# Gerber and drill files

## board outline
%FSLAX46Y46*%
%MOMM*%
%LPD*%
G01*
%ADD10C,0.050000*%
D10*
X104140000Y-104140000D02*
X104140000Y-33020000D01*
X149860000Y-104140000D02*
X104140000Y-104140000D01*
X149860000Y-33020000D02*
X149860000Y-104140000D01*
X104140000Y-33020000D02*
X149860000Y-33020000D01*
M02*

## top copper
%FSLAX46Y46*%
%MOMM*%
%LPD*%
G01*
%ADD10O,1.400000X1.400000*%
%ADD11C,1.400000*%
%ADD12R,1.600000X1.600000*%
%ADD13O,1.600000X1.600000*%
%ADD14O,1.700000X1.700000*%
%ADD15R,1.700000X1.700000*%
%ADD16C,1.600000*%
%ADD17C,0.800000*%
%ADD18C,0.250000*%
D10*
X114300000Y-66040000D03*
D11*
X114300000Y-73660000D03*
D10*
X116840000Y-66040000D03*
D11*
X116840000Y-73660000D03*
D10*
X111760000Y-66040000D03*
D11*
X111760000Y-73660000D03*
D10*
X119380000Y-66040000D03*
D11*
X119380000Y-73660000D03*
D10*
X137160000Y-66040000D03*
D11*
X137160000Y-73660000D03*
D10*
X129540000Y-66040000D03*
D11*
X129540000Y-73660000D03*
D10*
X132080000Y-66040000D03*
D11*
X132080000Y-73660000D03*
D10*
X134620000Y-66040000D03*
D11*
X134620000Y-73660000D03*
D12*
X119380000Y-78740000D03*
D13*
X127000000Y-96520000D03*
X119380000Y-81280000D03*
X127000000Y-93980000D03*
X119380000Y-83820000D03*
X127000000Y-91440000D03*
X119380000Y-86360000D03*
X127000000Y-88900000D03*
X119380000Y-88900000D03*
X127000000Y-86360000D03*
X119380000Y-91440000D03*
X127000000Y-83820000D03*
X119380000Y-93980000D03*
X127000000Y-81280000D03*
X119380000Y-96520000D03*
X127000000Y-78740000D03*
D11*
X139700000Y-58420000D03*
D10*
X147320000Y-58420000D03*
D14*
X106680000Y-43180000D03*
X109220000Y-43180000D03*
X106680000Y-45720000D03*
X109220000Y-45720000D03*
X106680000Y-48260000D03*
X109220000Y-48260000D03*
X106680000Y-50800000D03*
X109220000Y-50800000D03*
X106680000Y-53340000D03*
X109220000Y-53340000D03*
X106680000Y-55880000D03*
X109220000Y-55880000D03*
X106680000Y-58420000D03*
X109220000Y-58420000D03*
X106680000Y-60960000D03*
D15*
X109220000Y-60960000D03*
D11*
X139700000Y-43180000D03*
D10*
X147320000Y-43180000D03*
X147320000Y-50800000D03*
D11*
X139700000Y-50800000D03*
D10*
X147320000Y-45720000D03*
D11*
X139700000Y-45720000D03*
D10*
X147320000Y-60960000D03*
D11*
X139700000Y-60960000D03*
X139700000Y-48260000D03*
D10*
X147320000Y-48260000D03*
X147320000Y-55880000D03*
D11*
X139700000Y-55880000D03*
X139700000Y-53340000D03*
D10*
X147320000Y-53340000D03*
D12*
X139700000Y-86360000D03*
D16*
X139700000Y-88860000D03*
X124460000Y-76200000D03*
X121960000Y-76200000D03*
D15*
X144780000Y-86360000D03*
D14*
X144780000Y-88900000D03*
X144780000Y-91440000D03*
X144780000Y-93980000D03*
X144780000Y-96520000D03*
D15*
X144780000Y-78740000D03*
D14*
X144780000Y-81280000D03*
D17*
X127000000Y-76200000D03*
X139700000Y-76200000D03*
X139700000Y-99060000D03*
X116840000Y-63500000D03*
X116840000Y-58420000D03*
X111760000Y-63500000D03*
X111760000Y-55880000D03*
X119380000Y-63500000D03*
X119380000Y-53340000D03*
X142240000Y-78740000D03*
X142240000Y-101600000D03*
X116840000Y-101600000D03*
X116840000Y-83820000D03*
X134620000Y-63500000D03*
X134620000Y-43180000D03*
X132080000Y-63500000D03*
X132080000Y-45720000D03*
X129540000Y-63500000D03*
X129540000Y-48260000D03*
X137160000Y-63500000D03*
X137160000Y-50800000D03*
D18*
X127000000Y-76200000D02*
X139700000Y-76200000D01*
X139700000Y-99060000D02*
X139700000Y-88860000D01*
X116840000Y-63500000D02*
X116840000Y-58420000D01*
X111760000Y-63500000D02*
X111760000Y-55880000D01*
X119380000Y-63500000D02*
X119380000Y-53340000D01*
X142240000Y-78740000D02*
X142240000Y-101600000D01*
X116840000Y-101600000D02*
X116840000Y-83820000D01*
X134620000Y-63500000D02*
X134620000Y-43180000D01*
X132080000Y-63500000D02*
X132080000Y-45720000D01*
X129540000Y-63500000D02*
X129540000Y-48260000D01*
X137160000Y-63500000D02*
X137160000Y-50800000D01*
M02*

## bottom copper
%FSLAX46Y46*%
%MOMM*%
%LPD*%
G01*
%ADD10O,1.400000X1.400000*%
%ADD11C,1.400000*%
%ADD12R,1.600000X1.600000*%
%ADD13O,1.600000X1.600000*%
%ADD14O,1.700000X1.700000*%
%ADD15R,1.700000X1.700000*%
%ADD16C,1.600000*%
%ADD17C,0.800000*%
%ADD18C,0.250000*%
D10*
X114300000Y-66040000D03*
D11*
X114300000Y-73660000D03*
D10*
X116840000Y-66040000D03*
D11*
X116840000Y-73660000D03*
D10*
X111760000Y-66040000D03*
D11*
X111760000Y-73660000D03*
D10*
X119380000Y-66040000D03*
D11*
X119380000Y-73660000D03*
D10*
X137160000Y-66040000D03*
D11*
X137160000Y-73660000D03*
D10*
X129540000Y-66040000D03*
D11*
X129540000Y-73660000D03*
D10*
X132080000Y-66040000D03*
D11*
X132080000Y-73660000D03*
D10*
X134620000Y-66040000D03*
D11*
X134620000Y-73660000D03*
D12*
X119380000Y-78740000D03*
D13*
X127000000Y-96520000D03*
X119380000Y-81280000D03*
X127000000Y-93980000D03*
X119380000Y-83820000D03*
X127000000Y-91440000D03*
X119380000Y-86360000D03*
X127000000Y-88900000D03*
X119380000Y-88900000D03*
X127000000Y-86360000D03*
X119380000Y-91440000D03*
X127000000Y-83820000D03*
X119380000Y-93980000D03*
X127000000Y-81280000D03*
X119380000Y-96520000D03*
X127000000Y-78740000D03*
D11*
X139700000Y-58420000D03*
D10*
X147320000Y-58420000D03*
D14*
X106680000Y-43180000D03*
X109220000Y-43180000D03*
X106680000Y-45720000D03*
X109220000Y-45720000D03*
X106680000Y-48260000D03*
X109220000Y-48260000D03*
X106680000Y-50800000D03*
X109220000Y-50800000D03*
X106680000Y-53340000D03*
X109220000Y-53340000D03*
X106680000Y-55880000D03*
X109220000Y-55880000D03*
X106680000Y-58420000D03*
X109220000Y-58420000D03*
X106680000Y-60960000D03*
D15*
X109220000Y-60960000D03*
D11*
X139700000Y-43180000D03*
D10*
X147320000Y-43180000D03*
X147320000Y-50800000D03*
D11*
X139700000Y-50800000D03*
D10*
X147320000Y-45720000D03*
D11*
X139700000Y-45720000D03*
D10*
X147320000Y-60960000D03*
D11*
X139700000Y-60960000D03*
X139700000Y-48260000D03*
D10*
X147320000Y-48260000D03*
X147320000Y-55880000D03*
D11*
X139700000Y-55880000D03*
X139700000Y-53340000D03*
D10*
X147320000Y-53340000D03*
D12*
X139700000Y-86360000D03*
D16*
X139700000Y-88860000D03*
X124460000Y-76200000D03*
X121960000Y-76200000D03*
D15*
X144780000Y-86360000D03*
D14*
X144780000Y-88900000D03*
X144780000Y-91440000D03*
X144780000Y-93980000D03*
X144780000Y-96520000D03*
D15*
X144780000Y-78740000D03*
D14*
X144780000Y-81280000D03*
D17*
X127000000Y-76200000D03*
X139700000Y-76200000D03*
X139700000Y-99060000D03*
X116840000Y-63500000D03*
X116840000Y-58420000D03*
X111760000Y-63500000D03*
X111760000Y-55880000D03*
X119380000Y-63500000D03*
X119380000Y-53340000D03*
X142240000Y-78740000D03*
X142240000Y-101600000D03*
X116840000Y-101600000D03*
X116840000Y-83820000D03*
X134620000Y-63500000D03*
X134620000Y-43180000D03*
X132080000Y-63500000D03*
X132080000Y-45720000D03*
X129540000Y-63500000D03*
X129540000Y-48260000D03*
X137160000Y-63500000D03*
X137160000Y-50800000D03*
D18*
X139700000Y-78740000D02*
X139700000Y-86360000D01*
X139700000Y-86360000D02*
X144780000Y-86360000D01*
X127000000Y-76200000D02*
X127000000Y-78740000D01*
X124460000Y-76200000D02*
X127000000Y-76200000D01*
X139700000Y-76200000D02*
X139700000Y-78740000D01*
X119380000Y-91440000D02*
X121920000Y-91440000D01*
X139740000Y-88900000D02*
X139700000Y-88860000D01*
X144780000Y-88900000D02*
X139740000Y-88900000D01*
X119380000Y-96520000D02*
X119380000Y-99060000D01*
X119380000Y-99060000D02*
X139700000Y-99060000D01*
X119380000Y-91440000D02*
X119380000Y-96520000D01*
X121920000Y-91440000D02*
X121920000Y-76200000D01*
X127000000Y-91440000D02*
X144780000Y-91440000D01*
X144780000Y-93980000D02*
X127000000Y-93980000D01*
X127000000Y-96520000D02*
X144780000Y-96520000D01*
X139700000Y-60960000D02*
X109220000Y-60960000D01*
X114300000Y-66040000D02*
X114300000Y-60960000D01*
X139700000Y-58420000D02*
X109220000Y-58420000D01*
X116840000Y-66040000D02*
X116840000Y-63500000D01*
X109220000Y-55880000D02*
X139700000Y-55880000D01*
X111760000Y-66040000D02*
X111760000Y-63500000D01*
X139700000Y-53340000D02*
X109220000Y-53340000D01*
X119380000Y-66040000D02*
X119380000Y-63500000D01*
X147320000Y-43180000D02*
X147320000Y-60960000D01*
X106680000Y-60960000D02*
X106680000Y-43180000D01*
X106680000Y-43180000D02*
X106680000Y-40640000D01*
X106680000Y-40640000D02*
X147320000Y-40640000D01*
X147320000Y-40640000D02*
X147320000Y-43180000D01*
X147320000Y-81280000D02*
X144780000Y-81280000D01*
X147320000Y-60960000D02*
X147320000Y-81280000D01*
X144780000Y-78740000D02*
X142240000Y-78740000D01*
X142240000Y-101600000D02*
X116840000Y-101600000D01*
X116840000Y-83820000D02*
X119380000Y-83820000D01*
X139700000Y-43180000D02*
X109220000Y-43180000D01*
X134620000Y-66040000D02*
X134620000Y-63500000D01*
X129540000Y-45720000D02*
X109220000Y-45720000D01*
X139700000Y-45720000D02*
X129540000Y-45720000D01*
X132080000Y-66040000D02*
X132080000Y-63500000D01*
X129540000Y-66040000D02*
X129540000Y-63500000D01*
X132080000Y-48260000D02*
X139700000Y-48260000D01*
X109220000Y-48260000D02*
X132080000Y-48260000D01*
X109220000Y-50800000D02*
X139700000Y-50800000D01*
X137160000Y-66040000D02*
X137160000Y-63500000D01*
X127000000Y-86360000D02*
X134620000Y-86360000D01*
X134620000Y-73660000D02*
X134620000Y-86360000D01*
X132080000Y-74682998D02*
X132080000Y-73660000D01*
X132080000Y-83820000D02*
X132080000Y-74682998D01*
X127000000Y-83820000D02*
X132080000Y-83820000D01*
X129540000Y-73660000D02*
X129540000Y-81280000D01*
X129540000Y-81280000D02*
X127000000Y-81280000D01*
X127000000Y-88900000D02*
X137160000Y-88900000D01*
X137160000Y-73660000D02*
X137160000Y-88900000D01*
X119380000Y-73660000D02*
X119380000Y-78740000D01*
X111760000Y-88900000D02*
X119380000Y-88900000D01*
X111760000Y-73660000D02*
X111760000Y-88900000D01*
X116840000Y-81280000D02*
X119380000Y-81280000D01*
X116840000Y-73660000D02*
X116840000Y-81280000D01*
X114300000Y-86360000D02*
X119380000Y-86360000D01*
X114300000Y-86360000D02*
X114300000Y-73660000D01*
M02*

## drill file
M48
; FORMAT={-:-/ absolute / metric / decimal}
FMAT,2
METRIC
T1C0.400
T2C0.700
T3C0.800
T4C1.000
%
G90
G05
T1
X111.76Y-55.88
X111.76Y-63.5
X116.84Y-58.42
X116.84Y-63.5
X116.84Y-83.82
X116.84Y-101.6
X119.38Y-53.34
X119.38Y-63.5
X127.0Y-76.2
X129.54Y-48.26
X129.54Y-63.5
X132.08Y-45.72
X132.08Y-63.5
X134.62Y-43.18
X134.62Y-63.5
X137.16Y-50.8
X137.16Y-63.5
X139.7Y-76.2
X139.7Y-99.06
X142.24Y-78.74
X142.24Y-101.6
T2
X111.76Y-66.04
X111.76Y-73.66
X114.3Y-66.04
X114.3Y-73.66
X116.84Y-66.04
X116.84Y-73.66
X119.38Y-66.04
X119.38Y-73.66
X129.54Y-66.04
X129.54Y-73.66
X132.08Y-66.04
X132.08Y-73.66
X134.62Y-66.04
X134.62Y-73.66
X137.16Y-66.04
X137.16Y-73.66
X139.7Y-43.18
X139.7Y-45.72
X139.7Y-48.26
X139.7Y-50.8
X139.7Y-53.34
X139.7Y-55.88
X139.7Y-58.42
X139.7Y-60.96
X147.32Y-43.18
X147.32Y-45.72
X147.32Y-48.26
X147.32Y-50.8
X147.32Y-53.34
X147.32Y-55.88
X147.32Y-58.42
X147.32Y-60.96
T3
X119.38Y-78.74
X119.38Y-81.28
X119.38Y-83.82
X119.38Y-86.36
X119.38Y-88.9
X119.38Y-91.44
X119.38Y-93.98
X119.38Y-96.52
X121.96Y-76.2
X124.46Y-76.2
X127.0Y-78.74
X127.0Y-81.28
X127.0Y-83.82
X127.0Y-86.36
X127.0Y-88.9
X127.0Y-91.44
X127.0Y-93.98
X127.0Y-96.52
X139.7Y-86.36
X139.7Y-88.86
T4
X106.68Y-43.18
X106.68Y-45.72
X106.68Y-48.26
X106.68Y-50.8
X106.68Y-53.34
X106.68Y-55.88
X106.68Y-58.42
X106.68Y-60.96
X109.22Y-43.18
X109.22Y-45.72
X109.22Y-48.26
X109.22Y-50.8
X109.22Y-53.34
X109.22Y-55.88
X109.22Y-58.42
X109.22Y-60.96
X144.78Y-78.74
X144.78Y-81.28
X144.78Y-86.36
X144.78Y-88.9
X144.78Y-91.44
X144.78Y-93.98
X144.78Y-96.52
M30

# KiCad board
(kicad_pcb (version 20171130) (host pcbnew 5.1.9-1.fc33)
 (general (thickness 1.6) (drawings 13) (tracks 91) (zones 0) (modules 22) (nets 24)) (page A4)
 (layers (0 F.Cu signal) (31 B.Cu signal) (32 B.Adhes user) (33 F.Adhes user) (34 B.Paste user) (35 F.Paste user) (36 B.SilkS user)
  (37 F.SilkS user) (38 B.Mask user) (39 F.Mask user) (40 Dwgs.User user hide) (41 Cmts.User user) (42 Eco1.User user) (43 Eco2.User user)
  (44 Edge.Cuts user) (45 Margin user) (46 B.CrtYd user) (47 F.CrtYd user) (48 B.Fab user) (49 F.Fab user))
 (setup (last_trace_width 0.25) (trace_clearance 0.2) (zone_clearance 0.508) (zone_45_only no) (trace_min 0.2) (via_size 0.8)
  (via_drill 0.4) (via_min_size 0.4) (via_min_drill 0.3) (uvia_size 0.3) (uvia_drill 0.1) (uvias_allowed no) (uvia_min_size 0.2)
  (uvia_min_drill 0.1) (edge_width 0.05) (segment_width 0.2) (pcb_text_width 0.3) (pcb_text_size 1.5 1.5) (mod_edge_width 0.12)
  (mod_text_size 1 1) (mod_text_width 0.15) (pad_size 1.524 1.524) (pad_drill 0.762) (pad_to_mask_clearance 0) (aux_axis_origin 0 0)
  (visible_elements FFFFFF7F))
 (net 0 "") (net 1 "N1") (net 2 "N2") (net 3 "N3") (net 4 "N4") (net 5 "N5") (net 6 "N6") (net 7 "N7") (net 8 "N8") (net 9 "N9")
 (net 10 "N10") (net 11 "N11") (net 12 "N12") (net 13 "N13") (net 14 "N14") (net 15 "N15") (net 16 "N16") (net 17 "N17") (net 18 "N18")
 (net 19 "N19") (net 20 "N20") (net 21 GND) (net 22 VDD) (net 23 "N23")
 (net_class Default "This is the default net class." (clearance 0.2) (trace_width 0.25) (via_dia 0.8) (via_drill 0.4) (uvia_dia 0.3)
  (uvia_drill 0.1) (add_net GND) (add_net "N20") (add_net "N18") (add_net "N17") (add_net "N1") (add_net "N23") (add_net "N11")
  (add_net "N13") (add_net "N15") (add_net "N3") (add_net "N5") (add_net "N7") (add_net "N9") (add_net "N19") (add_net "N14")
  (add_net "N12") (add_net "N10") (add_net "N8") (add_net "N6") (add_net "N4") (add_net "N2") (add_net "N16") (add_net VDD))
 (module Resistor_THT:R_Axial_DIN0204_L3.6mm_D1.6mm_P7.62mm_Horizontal (layer F.Cu) (at 114.3 73.66 90)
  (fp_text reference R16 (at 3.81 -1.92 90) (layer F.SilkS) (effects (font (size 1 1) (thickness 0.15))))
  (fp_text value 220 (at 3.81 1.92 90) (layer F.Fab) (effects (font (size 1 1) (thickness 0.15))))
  (pad 2 thru_hole oval (at 7.62 0 90) (size 1.4 1.4) (drill 0.7) (layers *.Cu *.Mask) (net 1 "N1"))
  (pad 1 thru_hole circle (at 0 0 90) (size 1.4 1.4) (drill 0.7) (layers *.Cu *.Mask) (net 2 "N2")))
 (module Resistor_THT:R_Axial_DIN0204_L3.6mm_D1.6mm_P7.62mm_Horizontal (layer F.Cu) (at 116.84 73.66 90)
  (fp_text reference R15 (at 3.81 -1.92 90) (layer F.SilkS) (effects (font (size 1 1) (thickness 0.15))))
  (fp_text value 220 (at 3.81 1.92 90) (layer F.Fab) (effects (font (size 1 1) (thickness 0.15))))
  (pad 2 thru_hole oval (at 7.62 0 90) (size 1.4 1.4) (drill 0.7) (layers *.Cu *.Mask) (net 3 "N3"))
  (pad 1 thru_hole circle (at 0 0 90) (size 1.4 1.4) (drill 0.7) (layers *.Cu *.Mask) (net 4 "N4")))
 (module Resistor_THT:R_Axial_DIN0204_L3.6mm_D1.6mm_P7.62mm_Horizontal (layer F.Cu) (at 111.76 73.66 90)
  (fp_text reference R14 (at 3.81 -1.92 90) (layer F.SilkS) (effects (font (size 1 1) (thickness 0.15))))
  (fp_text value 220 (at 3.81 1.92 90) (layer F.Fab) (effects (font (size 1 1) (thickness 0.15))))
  (pad 2 thru_hole oval (at 7.62 0 90) (size 1.4 1.4) (drill 0.7) (layers *.Cu *.Mask) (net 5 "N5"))
  (pad 1 thru_hole circle (at 0 0 90) (size 1.4 1.4) (drill 0.7) (layers *.Cu *.Mask) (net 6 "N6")))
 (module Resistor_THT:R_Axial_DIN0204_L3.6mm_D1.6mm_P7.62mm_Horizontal (layer F.Cu) (at 119.38 73.66 90)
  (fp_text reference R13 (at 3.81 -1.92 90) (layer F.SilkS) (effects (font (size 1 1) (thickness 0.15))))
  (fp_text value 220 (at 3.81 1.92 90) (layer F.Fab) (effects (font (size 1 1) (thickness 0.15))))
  (pad 2 thru_hole oval (at 7.62 0 90) (size 1.4 1.4) (drill 0.7) (layers *.Cu *.Mask) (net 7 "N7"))
  (pad 1 thru_hole circle (at 0 0 90) (size 1.4 1.4) (drill 0.7) (layers *.Cu *.Mask) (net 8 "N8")))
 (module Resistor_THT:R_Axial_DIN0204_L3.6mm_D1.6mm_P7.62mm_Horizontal (layer F.Cu) (at 137.16 73.66 90)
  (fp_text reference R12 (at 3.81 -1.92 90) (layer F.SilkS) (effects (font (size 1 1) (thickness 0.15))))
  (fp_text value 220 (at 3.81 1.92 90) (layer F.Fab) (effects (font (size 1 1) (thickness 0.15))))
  (pad 2 thru_hole oval (at 7.62 0 90) (size 1.4 1.4) (drill 0.7) (layers *.Cu *.Mask) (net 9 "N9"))
  (pad 1 thru_hole circle (at 0 0 90) (size 1.4 1.4) (drill 0.7) (layers *.Cu *.Mask) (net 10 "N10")))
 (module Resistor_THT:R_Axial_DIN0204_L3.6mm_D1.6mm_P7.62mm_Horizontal (layer F.Cu) (at 129.54 73.66 90)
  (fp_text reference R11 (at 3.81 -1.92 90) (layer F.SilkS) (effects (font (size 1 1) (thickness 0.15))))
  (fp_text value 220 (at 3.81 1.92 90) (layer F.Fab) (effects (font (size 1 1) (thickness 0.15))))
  (pad 2 thru_hole oval (at 7.62 0 90) (size 1.4 1.4) (drill 0.7) (layers *.Cu *.Mask) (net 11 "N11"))
  (pad 1 thru_hole circle (at 0 0 90) (size 1.4 1.4) (drill 0.7) (layers *.Cu *.Mask) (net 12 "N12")))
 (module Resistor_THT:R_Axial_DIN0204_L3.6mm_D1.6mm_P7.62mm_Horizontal (layer F.Cu) (at 132.08 73.66 90)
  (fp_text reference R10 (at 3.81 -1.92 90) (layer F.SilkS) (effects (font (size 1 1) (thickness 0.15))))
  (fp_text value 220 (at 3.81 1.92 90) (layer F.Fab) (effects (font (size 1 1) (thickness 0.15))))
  (pad 2 thru_hole oval (at 7.62 0 90) (size 1.4 1.4) (drill 0.7) (layers *.Cu *.Mask) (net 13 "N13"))
  (pad 1 thru_hole circle (at 0 0 90) (size 1.4 1.4) (drill 0.7) (layers *.Cu *.Mask) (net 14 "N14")))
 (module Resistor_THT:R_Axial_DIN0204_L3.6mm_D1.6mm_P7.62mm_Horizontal (layer F.Cu) (at 134.62 73.66 90)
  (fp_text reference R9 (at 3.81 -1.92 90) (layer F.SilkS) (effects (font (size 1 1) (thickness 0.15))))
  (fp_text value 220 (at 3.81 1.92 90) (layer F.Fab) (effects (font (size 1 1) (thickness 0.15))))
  (pad 2 thru_hole oval (at 7.62 0 90) (size 1.4 1.4) (drill 0.7) (layers *.Cu *.Mask) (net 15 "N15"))
  (pad 1 thru_hole circle (at 0 0 90) (size 1.4 1.4) (drill 0.7) (layers *.Cu *.Mask) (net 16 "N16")))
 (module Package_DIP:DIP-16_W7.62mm (layer F.Cu) (at 119.38 78.74)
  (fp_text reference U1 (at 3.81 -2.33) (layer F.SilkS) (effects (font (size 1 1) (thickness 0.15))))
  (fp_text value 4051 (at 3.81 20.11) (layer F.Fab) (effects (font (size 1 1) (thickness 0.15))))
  (pad 1 thru_hole rect (at 0 0) (size 1.6 1.6) (drill 0.8) (layers *.Cu *.Mask) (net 8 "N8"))
  (pad 9 thru_hole oval (at 7.62 17.78) (size 1.6 1.6) (drill 0.8) (layers *.Cu *.Mask) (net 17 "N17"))
  (pad 2 thru_hole oval (at 0 2.54) (size 1.6 1.6) (drill 0.8) (layers *.Cu *.Mask) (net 4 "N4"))
  (pad 10 thru_hole oval (at 7.62 15.24) (size 1.6 1.6) (drill 0.8) (layers *.Cu *.Mask) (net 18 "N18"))
  (pad 3 thru_hole oval (at 0 5.08) (size 1.6 1.6) (drill 0.8) (layers *.Cu *.Mask) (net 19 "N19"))
  (pad 11 thru_hole oval (at 7.62 12.7) (size 1.6 1.6) (drill 0.8) (layers *.Cu *.Mask) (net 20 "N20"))
  (pad 4 thru_hole oval (at 0 7.62) (size 1.6 1.6) (drill 0.8) (layers *.Cu *.Mask) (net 2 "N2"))
  (pad 12 thru_hole oval (at 7.62 10.16) (size 1.6 1.6) (drill 0.8) (layers *.Cu *.Mask) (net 10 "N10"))
  (pad 5 thru_hole oval (at 0 10.16) (size 1.6 1.6) (drill 0.8) (layers *.Cu *.Mask) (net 6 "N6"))
  (pad 13 thru_hole oval (at 7.62 7.62) (size 1.6 1.6) (drill 0.8) (layers *.Cu *.Mask) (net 16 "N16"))
  (pad 6 thru_hole oval (at 0 12.7) (size 1.6 1.6) (drill 0.8) (layers *.Cu *.Mask) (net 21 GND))
  (pad 14 thru_hole oval (at 7.62 5.08) (size 1.6 1.6) (drill 0.8) (layers *.Cu *.Mask) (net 14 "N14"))
  (pad 7 thru_hole oval (at 0 15.24) (size 1.6 1.6) (drill 0.8) (layers *.Cu *.Mask) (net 21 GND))
  (pad 15 thru_hole oval (at 7.62 2.54) (size 1.6 1.6) (drill 0.8) (layers *.Cu *.Mask) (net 12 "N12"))
  (pad 8 thru_hole oval (at 0 17.78) (size 1.6 1.6) (drill 0.8) (layers *.Cu *.Mask) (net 21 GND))
  (pad 16 thru_hole oval (at 7.62 0) (size 1.6 1.6) (drill 0.8) (layers *.Cu *.Mask) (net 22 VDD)))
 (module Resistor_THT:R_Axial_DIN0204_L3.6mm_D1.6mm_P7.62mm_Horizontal (layer F.Cu) (at 139.7 58.42)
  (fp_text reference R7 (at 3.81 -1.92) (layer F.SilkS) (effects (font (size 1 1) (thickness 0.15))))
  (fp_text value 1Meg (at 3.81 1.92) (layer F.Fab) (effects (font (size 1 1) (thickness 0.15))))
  (pad 1 thru_hole circle (at 0 0) (size 1.4 1.4) (drill 0.7) (layers *.Cu *.Mask) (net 3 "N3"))
  (pad 2 thru_hole oval (at 7.62 0) (size 1.4 1.4) (drill 0.7) (layers *.Cu *.Mask) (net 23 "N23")))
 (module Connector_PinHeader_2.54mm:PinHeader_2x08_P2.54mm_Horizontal (layer F.Cu) (at 109.22 60.96 180)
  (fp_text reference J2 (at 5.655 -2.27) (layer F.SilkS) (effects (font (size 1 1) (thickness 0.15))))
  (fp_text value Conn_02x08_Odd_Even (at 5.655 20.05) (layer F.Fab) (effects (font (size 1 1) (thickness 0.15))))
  (pad 16 thru_hole oval (at 2.54 17.78 180) (size 1.7 1.7) (drill 1) (layers *.Cu *.Mask) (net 23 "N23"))
  (pad 15 thru_hole oval (at 0 17.78 180) (size 1.7 1.7) (drill 1) (layers *.Cu *.Mask) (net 15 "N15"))
  (pad 14 thru_hole oval (at 2.54 15.24 180) (size 1.7 1.7) (drill 1) (layers *.Cu *.Mask) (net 23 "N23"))
  (pad 13 thru_hole oval (at 0 15.24 180) (size 1.7 1.7) (drill 1) (layers *.Cu *.Mask) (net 13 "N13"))
  (pad 12 thru_hole oval (at 2.54 12.7 180) (size 1.7 1.7) (drill 1) (layers *.Cu *.Mask) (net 23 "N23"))
  (pad 11 thru_hole oval (at 0 12.7 180) (size 1.7 1.7) (drill 1) (layers *.Cu *.Mask) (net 11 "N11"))
  (pad 10 thru_hole oval (at 2.54 10.16 180) (size 1.7 1.7) (drill 1) (layers *.Cu *.Mask) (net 23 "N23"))
  (pad 9 thru_hole oval (at 0 10.16 180) (size 1.7 1.7) (drill 1) (layers *.Cu *.Mask) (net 9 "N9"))
  (pad 8 thru_hole oval (at 2.54 7.62 180) (size 1.7 1.7) (drill 1) (layers *.Cu *.Mask) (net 23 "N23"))
  (pad 7 thru_hole oval (at 0 7.62 180) (size 1.7 1.7) (drill 1) (layers *.Cu *.Mask) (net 7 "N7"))
  (pad 6 thru_hole oval (at 2.54 5.08 180) (size 1.7 1.7) (drill 1) (layers *.Cu *.Mask) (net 23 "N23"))
  (pad 5 thru_hole oval (at 0 5.08 180) (size 1.7 1.7) (drill 1) (layers *.Cu *.Mask) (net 5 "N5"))
  (pad 4 thru_hole oval (at 2.54 2.54 180) (size 1.7 1.7) (drill 1) (layers *.Cu *.Mask) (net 23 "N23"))
  (pad 3 thru_hole oval (at 0 2.54 180) (size 1.7 1.7) (drill 1) (layers *.Cu *.Mask) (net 3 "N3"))
  (pad 2 thru_hole oval (at 2.54 0 180) (size 1.7 1.7) (drill 1) (layers *.Cu *.Mask) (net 23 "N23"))
  (pad 1 thru_hole rect (at 0 0 180) (size 1.7 1.7) (drill 1) (layers *.Cu *.Mask) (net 1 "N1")))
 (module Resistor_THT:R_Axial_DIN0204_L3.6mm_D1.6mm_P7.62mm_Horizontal (layer F.Cu) (at 139.7 43.18)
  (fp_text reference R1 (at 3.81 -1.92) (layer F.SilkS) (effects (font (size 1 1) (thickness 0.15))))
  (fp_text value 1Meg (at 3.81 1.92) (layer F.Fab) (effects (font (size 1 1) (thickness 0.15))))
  (pad 1 thru_hole circle (at 0 0) (size 1.4 1.4) (drill 0.7) (layers *.Cu *.Mask) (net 15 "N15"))
  (pad 2 thru_hole oval (at 7.62 0) (size 1.4 1.4) (drill 0.7) (layers *.Cu *.Mask) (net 23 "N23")))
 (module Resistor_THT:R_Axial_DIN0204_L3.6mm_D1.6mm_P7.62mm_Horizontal (layer F.Cu) (at 139.7 50.8)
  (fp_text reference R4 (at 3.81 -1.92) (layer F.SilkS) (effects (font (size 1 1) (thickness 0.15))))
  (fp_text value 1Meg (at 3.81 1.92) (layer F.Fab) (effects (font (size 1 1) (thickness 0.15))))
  (pad 2 thru_hole oval (at 7.62 0) (size 1.4 1.4) (drill 0.7) (layers *.Cu *.Mask) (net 23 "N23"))
  (pad 1 thru_hole circle (at 0 0) (size 1.4 1.4) (drill 0.7) (layers *.Cu *.Mask) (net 9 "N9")))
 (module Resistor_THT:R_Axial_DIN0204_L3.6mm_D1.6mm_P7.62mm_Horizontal (layer F.Cu) (at 139.7 45.72)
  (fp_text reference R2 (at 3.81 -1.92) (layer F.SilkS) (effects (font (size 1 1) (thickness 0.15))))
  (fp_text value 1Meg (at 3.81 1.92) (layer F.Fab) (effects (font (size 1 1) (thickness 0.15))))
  (pad 2 thru_hole oval (at 7.62 0) (size 1.4 1.4) (drill 0.7) (layers *.Cu *.Mask) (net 23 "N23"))
  (pad 1 thru_hole circle (at 0 0) (size 1.4 1.4) (drill 0.7) (layers *.Cu *.Mask) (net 13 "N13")))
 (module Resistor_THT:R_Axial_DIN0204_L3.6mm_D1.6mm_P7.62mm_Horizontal (layer F.Cu) (at 139.7 60.96)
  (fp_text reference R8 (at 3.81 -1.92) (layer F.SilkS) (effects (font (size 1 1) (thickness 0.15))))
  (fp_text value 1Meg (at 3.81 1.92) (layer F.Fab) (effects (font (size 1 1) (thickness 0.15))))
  (pad 2 thru_hole oval (at 7.62 0) (size 1.4 1.4) (drill 0.7) (layers *.Cu *.Mask) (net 23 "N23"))
  (pad 1 thru_hole circle (at 0 0) (size 1.4 1.4) (drill 0.7) (layers *.Cu *.Mask) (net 1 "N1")))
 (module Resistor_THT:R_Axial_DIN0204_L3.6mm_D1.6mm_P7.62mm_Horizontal (layer F.Cu) (at 139.7 48.26)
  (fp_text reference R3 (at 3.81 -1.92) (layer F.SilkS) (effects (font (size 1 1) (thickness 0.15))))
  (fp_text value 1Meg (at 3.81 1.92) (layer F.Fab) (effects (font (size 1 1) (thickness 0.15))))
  (pad 1 thru_hole circle (at 0 0) (size 1.4 1.4) (drill 0.7) (layers *.Cu *.Mask) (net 11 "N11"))
  (pad 2 thru_hole oval (at 7.62 0) (size 1.4 1.4) (drill 0.7) (layers *.Cu *.Mask) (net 23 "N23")))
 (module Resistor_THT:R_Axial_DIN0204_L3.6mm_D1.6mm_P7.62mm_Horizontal (layer F.Cu) (at 139.7 55.88)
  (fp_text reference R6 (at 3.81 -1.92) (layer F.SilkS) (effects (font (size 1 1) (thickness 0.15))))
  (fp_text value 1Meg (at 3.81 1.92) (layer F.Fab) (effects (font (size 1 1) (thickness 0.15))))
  (pad 2 thru_hole oval (at 7.62 0) (size 1.4 1.4) (drill 0.7) (layers *.Cu *.Mask) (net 23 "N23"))
  (pad 1 thru_hole circle (at 0 0) (size 1.4 1.4) (drill 0.7) (layers *.Cu *.Mask) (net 5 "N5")))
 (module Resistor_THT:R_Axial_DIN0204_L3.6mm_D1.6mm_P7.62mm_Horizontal (layer F.Cu) (at 139.7 53.34)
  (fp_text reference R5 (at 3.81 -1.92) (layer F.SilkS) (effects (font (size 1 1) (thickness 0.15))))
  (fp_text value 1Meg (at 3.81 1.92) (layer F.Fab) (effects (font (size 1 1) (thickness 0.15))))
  (pad 1 thru_hole circle (at 0 0) (size 1.4 1.4) (drill 0.7) (layers *.Cu *.Mask) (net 7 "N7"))
  (pad 2 thru_hole oval (at 7.62 0) (size 1.4 1.4) (drill 0.7) (layers *.Cu *.Mask) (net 23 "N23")))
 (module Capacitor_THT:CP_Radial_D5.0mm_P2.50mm (layer F.Cu) (at 139.7 86.36 270)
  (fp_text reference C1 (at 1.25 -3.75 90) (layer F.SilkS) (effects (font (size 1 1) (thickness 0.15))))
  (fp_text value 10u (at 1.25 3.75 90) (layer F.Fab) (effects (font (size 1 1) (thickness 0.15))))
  (pad 1 thru_hole rect (at 0 0 270) (size 1.6 1.6) (drill 0.8) (layers *.Cu *.Mask) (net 22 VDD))
  (pad 2 thru_hole circle (at 2.5 0 270) (size 1.6 1.6) (drill 0.8) (layers *.Cu *.Mask) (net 21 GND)))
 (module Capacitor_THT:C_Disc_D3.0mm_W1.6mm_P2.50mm (layer F.Cu) (at 124.46 76.2 180)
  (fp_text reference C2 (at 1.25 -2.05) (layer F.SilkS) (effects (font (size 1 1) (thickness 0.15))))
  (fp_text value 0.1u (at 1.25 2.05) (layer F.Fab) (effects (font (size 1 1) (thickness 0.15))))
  (pad 1 thru_hole circle (at 0 0 180) (size 1.6 1.6) (drill 0.8) (layers *.Cu *.Mask) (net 22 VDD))
  (pad 2 thru_hole circle (at 2.5 0 180) (size 1.6 1.6) (drill 0.8) (layers *.Cu *.Mask) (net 21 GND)))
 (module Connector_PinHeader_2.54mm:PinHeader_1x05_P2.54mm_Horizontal (layer F.Cu) (at 144.78 86.36)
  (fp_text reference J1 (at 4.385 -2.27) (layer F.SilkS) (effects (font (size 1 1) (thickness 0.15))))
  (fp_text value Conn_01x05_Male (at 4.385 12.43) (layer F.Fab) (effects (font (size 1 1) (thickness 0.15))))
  (pad 1 thru_hole rect (at 0 0) (size 1.7 1.7) (drill 1) (layers *.Cu *.Mask) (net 22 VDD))
  (pad 2 thru_hole oval (at 0 2.54) (size 1.7 1.7) (drill 1) (layers *.Cu *.Mask) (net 21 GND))
  (pad 3 thru_hole oval (at 0 5.08) (size 1.7 1.7) (drill 1) (layers *.Cu *.Mask) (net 20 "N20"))
  (pad 4 thru_hole oval (at 0 7.62) (size 1.7 1.7) (drill 1) (layers *.Cu *.Mask) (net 18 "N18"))
  (pad 5 thru_hole oval (at 0 10.16) (size 1.7 1.7) (drill 1) (layers *.Cu *.Mask) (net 17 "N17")))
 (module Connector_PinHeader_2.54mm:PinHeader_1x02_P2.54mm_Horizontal (layer F.Cu) (at 144.78 78.74)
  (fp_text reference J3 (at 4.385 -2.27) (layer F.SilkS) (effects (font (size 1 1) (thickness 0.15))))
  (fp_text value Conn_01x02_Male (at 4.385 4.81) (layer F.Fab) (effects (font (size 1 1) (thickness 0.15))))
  (pad 1 thru_hole rect (at 0 0) (size 1.7 1.7) (drill 1) (layers *.Cu *.Mask) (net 19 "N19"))
  (pad 2 thru_hole oval (at 0 2.54) (size 1.7 1.7) (drill 1) (layers *.Cu *.Mask) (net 23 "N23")))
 (gr_line (start 104.14 104.14) (end 104.14 33.02) (layer Edge.Cuts) (width 0.05))
 (gr_line (start 149.86 104.14) (end 104.14 104.14) (layer Edge.Cuts) (width 0.05))
 (gr_line (start 149.86 33.02) (end 149.86 104.14) (layer Edge.Cuts) (width 0.05))
 (gr_line (start 104.14 33.02) (end 149.86 33.02) (layer Edge.Cuts) (width 0.05))
 (segment (start 139.7 78.74) (end 139.7 86.36) (width 0.25) (layer B.Cu) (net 22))
 (segment (start 139.7 86.36) (end 144.78 86.36) (width 0.25) (layer B.Cu) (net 22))
 (segment (start 127 76.2) (end 127 78.74) (width 0.25) (layer B.Cu) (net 22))
 (via (at 127 76.2) (size 0.8) (drill 0.4) (layers F.Cu B.Cu) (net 22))
 (segment (start 124.46 76.2) (end 127 76.2) (width 0.25) (layer B.Cu) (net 22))
 (via (at 139.7 76.2) (size 0.8) (drill 0.4) (layers F.Cu B.Cu) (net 22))
 (segment (start 127 76.2) (end 139.7 76.2) (width 0.25) (layer F.Cu) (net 22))
 (segment (start 139.7 76.2) (end 139.7 78.74) (width 0.25) (layer B.Cu) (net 22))
 (segment (start 119.38 91.44) (end 121.92 91.44) (width 0.25) (layer B.Cu) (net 21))
 (segment (start 139.74 88.9) (end 139.7 88.86) (width 0.25) (layer B.Cu) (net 21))
 (segment (start 144.78 88.9) (end 139.74 88.9) (width 0.25) (layer B.Cu) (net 21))
 (segment (start 119.38 96.52) (end 119.38 99.06) (width 0.25) (layer B.Cu) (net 21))
 (via (at 139.7 99.06) (size 0.8) (drill 0.4) (layers F.Cu B.Cu) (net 21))
 (segment (start 119.38 99.06) (end 139.7 99.06) (width 0.25) (layer B.Cu) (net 21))
 (segment (start 139.7 99.06) (end 139.7 88.86) (width 0.25) (layer F.Cu) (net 21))
 (segment (start 119.38 91.44) (end 119.38 96.52) (width 0.25) (layer B.Cu) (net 21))
 (segment (start 121.92 91.44) (end 121.92 76.2) (width 0.25) (layer B.Cu) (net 21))
 (segment (start 127 91.44) (end 144.78 91.44) (width 0.25) (layer B.Cu) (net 20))
 (segment (start 144.78 93.98) (end 127 93.98) (width 0.25) (layer B.Cu) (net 18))
 (segment (start 127 96.52) (end 144.78 96.52) (width 0.25) (layer B.Cu) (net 17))
 (segment (start 139.7 60.96) (end 109.22 60.96) (width 0.25) (layer B.Cu) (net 1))
 (segment (start 114.3 66.04) (end 114.3 60.96) (width 0.25) (layer B.Cu) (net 1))
 (segment (start 139.7 58.42) (end 109.22 58.42) (width 0.25) (layer B.Cu) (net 3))
 (via (at 116.84 63.5) (size 0.8) (drill 0.4) (layers F.Cu B.Cu) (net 3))
 (segment (start 116.84 66.04) (end 116.84 63.5) (width 0.25) (layer B.Cu) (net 3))
 (via (at 116.84 58.42) (size 0.8) (drill 0.4) (layers F.Cu B.Cu) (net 3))
 (segment (start 116.84 63.5) (end 116.84 58.42) (width 0.25) (layer F.Cu) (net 3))
 (segment (start 109.22 55.88) (end 139.7 55.88) (width 0.25) (layer B.Cu) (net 5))
 (via (at 111.76 63.5) (size 0.8) (drill 0.4) (layers F.Cu B.Cu) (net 5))
 (segment (start 111.76 66.04) (end 111.76 63.5) (width 0.25) (layer B.Cu) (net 5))
 (segment (start 111.76 63.5) (end 111.76 55.88) (width 0.25) (layer F.Cu) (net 5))
 (via (at 111.76 55.88) (size 0.8) (drill 0.4) (layers F.Cu B.Cu) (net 5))
 (segment (start 139.7 53.34) (end 109.22 53.34) (width 0.25) (layer B.Cu) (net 7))
 (via (at 119.38 63.5) (size 0.8) (drill 0.4) (layers F.Cu B.Cu) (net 7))
 (segment (start 119.38 66.04) (end 119.38 63.5) (width 0.25) (layer B.Cu) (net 7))
 (via (at 119.38 53.34) (size 0.8) (drill 0.4) (layers F.Cu B.Cu) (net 7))
 (segment (start 119.38 63.5) (end 119.38 53.34) (width 0.25) (layer F.Cu) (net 7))
 (segment (start 147.32 43.18) (end 147.32 60.96) (width 0.25) (layer B.Cu) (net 23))
 (segment (start 106.68 60.96) (end 106.68 43.18) (width 0.25) (layer B.Cu) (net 23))
 (segment (start 106.68 43.18) (end 106.68 40.64) (width 0.25) (layer B.Cu) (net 23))
 (segment (start 106.68 40.64) (end 147.32 40.64) (width 0.25) (layer B.Cu) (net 23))
 (segment (start 147.32 40.64) (end 147.32 43.18) (width 0.25) (layer B.Cu) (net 23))
 (segment (start 147.32 81.28) (end 144.78 81.28) (width 0.25) (layer B.Cu) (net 23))
 (segment (start 147.32 60.96) (end 147.32 81.28) (width 0.25) (layer B.Cu) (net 23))
 (via (at 142.24 78.74) (size 0.8) (drill 0.4) (layers F.Cu B.Cu) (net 19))
 (segment (start 144.78 78.74) (end 142.24 78.74) (width 0.25) (layer B.Cu) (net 19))
 (via (at 142.24 101.6) (size 0.8) (drill 0.4) (layers F.Cu B.Cu) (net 19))
 (segment (start 142.24 78.74) (end 142.24 101.6) (width 0.25) (layer F.Cu) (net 19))
 (via (at 116.84 101.6) (size 0.8) (drill 0.4) (layers F.Cu B.Cu) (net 19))
 (segment (start 142.24 101.6) (end 116.84 101.6) (width 0.25) (layer B.Cu) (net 19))
 (via (at 116.84 83.82) (size 0.8) (drill 0.4) (layers F.Cu B.Cu) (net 19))
 (segment (start 116.84 101.6) (end 116.84 83.82) (width 0.25) (layer F.Cu) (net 19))
 (segment (start 116.84 83.82) (end 119.38 83.82) (width 0.25) (layer B.Cu) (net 19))
 (segment (start 139.7 43.18) (end 109.22 43.18) (width 0.25) (layer B.Cu) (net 15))
 (via (at 134.62 63.5) (size 0.8) (drill 0.4) (layers F.Cu B.Cu) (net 15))
 (segment (start 134.62 66.04) (end 134.62 63.5) (width 0.25) (layer B.Cu) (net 15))
 (via (at 134.62 43.18) (size 0.8) (drill 0.4) (layers F.Cu B.Cu) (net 15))
 (segment (start 134.62 63.5) (end 134.62 43.18) (width 0.25) (layer F.Cu) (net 15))
 (segment (start 129.54 45.72) (end 109.22 45.72) (width 0.25) (layer B.Cu) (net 13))
 (segment (start 139.7 45.72) (end 129.54 45.72) (width 0.25) (layer B.Cu) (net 13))
 (via (at 132.08 63.5) (size 0.8) (drill 0.4) (layers F.Cu B.Cu) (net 13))
 (segment (start 132.08 66.04) (end 132.08 63.5) (width 0.25) (layer B.Cu) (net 13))
 (via (at 132.08 45.72) (size 0.8) (drill 0.4) (layers F.Cu B.Cu) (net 13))
 (segment (start 132.08 63.5) (end 132.08 45.72) (width 0.25) (layer F.Cu) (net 13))
 (via (at 129.54 63.5) (size 0.8) (drill 0.4) (layers F.Cu B.Cu) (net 11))
 (segment (start 129.54 66.04) (end 129.54 63.5) (width 0.25) (layer B.Cu) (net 11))
 (segment (start 132.08 48.26) (end 139.7 48.26) (width 0.25) (layer B.Cu) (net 11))
 (segment (start 109.22 48.26) (end 132.08 48.26) (width 0.25) (layer B.Cu) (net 11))
 (via (at 129.54 48.26) (size 0.8) (drill 0.4) (layers F.Cu B.Cu) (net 11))
 (segment (start 129.54 63.5) (end 129.54 48.26) (width 0.25) (layer F.Cu) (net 11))
 (segment (start 109.22 50.8) (end 139.7 50.8) (width 0.25) (layer B.Cu) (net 9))
 (via (at 137.16 63.5) (size 0.8) (drill 0.4) (layers F.Cu B.Cu) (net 9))
 (segment (start 137.16 66.04) (end 137.16 63.5) (width 0.25) (layer B.Cu) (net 9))
 (via (at 137.16 50.8) (size 0.8) (drill 0.4) (layers F.Cu B.Cu) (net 9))
 (segment (start 137.16 63.5) (end 137.16 50.8) (width 0.25) (layer F.Cu) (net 9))
 (segment (start 127 86.36) (end 134.62 86.36) (width 0.25) (layer B.Cu) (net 16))
 (segment (start 134.62 73.66) (end 134.62 86.36) (width 0.25) (layer B.Cu) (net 16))
 (segment (start 132.08 74.682998) (end 132.08 73.66) (width 0.25) (layer B.Cu) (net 14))
 (segment (start 132.08 83.82) (end 132.08 74.682998) (width 0.25) (layer B.Cu) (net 14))
 (segment (start 127 83.82) (end 132.08 83.82) (width 0.25) (layer B.Cu) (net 14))
 (segment (start 129.54 73.66) (end 129.54 81.28) (width 0.25) (layer B.Cu) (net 12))
 (segment (start 129.54 81.28) (end 127 81.28) (width 0.25) (layer B.Cu) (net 12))
 (segment (start 127 88.9) (end 137.16 88.9) (width 0.25) (layer B.Cu) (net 10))
 (segment (start 137.16 73.66) (end 137.16 88.9) (width 0.25) (layer B.Cu) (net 10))
 (segment (start 119.38 73.66) (end 119.38 78.74) (width 0.25) (layer B.Cu) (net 8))
 (segment (start 111.76 88.9) (end 119.38 88.9) (width 0.25) (layer B.Cu) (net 6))
 (segment (start 111.76 73.66) (end 111.76 88.9) (width 0.25) (layer B.Cu) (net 6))
 (segment (start 116.84 81.28) (end 119.38 81.28) (width 0.25) (layer B.Cu) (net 4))
 (segment (start 116.84 73.66) (end 116.84 81.28) (width 0.25) (layer B.Cu) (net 4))
 (segment (start 114.3 86.36) (end 119.38 86.36) (width 0.25) (layer B.Cu) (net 2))
 (segment (start 114.3 86.36) (end 114.3 73.66) (width 0.25) (layer B.Cu) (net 2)))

